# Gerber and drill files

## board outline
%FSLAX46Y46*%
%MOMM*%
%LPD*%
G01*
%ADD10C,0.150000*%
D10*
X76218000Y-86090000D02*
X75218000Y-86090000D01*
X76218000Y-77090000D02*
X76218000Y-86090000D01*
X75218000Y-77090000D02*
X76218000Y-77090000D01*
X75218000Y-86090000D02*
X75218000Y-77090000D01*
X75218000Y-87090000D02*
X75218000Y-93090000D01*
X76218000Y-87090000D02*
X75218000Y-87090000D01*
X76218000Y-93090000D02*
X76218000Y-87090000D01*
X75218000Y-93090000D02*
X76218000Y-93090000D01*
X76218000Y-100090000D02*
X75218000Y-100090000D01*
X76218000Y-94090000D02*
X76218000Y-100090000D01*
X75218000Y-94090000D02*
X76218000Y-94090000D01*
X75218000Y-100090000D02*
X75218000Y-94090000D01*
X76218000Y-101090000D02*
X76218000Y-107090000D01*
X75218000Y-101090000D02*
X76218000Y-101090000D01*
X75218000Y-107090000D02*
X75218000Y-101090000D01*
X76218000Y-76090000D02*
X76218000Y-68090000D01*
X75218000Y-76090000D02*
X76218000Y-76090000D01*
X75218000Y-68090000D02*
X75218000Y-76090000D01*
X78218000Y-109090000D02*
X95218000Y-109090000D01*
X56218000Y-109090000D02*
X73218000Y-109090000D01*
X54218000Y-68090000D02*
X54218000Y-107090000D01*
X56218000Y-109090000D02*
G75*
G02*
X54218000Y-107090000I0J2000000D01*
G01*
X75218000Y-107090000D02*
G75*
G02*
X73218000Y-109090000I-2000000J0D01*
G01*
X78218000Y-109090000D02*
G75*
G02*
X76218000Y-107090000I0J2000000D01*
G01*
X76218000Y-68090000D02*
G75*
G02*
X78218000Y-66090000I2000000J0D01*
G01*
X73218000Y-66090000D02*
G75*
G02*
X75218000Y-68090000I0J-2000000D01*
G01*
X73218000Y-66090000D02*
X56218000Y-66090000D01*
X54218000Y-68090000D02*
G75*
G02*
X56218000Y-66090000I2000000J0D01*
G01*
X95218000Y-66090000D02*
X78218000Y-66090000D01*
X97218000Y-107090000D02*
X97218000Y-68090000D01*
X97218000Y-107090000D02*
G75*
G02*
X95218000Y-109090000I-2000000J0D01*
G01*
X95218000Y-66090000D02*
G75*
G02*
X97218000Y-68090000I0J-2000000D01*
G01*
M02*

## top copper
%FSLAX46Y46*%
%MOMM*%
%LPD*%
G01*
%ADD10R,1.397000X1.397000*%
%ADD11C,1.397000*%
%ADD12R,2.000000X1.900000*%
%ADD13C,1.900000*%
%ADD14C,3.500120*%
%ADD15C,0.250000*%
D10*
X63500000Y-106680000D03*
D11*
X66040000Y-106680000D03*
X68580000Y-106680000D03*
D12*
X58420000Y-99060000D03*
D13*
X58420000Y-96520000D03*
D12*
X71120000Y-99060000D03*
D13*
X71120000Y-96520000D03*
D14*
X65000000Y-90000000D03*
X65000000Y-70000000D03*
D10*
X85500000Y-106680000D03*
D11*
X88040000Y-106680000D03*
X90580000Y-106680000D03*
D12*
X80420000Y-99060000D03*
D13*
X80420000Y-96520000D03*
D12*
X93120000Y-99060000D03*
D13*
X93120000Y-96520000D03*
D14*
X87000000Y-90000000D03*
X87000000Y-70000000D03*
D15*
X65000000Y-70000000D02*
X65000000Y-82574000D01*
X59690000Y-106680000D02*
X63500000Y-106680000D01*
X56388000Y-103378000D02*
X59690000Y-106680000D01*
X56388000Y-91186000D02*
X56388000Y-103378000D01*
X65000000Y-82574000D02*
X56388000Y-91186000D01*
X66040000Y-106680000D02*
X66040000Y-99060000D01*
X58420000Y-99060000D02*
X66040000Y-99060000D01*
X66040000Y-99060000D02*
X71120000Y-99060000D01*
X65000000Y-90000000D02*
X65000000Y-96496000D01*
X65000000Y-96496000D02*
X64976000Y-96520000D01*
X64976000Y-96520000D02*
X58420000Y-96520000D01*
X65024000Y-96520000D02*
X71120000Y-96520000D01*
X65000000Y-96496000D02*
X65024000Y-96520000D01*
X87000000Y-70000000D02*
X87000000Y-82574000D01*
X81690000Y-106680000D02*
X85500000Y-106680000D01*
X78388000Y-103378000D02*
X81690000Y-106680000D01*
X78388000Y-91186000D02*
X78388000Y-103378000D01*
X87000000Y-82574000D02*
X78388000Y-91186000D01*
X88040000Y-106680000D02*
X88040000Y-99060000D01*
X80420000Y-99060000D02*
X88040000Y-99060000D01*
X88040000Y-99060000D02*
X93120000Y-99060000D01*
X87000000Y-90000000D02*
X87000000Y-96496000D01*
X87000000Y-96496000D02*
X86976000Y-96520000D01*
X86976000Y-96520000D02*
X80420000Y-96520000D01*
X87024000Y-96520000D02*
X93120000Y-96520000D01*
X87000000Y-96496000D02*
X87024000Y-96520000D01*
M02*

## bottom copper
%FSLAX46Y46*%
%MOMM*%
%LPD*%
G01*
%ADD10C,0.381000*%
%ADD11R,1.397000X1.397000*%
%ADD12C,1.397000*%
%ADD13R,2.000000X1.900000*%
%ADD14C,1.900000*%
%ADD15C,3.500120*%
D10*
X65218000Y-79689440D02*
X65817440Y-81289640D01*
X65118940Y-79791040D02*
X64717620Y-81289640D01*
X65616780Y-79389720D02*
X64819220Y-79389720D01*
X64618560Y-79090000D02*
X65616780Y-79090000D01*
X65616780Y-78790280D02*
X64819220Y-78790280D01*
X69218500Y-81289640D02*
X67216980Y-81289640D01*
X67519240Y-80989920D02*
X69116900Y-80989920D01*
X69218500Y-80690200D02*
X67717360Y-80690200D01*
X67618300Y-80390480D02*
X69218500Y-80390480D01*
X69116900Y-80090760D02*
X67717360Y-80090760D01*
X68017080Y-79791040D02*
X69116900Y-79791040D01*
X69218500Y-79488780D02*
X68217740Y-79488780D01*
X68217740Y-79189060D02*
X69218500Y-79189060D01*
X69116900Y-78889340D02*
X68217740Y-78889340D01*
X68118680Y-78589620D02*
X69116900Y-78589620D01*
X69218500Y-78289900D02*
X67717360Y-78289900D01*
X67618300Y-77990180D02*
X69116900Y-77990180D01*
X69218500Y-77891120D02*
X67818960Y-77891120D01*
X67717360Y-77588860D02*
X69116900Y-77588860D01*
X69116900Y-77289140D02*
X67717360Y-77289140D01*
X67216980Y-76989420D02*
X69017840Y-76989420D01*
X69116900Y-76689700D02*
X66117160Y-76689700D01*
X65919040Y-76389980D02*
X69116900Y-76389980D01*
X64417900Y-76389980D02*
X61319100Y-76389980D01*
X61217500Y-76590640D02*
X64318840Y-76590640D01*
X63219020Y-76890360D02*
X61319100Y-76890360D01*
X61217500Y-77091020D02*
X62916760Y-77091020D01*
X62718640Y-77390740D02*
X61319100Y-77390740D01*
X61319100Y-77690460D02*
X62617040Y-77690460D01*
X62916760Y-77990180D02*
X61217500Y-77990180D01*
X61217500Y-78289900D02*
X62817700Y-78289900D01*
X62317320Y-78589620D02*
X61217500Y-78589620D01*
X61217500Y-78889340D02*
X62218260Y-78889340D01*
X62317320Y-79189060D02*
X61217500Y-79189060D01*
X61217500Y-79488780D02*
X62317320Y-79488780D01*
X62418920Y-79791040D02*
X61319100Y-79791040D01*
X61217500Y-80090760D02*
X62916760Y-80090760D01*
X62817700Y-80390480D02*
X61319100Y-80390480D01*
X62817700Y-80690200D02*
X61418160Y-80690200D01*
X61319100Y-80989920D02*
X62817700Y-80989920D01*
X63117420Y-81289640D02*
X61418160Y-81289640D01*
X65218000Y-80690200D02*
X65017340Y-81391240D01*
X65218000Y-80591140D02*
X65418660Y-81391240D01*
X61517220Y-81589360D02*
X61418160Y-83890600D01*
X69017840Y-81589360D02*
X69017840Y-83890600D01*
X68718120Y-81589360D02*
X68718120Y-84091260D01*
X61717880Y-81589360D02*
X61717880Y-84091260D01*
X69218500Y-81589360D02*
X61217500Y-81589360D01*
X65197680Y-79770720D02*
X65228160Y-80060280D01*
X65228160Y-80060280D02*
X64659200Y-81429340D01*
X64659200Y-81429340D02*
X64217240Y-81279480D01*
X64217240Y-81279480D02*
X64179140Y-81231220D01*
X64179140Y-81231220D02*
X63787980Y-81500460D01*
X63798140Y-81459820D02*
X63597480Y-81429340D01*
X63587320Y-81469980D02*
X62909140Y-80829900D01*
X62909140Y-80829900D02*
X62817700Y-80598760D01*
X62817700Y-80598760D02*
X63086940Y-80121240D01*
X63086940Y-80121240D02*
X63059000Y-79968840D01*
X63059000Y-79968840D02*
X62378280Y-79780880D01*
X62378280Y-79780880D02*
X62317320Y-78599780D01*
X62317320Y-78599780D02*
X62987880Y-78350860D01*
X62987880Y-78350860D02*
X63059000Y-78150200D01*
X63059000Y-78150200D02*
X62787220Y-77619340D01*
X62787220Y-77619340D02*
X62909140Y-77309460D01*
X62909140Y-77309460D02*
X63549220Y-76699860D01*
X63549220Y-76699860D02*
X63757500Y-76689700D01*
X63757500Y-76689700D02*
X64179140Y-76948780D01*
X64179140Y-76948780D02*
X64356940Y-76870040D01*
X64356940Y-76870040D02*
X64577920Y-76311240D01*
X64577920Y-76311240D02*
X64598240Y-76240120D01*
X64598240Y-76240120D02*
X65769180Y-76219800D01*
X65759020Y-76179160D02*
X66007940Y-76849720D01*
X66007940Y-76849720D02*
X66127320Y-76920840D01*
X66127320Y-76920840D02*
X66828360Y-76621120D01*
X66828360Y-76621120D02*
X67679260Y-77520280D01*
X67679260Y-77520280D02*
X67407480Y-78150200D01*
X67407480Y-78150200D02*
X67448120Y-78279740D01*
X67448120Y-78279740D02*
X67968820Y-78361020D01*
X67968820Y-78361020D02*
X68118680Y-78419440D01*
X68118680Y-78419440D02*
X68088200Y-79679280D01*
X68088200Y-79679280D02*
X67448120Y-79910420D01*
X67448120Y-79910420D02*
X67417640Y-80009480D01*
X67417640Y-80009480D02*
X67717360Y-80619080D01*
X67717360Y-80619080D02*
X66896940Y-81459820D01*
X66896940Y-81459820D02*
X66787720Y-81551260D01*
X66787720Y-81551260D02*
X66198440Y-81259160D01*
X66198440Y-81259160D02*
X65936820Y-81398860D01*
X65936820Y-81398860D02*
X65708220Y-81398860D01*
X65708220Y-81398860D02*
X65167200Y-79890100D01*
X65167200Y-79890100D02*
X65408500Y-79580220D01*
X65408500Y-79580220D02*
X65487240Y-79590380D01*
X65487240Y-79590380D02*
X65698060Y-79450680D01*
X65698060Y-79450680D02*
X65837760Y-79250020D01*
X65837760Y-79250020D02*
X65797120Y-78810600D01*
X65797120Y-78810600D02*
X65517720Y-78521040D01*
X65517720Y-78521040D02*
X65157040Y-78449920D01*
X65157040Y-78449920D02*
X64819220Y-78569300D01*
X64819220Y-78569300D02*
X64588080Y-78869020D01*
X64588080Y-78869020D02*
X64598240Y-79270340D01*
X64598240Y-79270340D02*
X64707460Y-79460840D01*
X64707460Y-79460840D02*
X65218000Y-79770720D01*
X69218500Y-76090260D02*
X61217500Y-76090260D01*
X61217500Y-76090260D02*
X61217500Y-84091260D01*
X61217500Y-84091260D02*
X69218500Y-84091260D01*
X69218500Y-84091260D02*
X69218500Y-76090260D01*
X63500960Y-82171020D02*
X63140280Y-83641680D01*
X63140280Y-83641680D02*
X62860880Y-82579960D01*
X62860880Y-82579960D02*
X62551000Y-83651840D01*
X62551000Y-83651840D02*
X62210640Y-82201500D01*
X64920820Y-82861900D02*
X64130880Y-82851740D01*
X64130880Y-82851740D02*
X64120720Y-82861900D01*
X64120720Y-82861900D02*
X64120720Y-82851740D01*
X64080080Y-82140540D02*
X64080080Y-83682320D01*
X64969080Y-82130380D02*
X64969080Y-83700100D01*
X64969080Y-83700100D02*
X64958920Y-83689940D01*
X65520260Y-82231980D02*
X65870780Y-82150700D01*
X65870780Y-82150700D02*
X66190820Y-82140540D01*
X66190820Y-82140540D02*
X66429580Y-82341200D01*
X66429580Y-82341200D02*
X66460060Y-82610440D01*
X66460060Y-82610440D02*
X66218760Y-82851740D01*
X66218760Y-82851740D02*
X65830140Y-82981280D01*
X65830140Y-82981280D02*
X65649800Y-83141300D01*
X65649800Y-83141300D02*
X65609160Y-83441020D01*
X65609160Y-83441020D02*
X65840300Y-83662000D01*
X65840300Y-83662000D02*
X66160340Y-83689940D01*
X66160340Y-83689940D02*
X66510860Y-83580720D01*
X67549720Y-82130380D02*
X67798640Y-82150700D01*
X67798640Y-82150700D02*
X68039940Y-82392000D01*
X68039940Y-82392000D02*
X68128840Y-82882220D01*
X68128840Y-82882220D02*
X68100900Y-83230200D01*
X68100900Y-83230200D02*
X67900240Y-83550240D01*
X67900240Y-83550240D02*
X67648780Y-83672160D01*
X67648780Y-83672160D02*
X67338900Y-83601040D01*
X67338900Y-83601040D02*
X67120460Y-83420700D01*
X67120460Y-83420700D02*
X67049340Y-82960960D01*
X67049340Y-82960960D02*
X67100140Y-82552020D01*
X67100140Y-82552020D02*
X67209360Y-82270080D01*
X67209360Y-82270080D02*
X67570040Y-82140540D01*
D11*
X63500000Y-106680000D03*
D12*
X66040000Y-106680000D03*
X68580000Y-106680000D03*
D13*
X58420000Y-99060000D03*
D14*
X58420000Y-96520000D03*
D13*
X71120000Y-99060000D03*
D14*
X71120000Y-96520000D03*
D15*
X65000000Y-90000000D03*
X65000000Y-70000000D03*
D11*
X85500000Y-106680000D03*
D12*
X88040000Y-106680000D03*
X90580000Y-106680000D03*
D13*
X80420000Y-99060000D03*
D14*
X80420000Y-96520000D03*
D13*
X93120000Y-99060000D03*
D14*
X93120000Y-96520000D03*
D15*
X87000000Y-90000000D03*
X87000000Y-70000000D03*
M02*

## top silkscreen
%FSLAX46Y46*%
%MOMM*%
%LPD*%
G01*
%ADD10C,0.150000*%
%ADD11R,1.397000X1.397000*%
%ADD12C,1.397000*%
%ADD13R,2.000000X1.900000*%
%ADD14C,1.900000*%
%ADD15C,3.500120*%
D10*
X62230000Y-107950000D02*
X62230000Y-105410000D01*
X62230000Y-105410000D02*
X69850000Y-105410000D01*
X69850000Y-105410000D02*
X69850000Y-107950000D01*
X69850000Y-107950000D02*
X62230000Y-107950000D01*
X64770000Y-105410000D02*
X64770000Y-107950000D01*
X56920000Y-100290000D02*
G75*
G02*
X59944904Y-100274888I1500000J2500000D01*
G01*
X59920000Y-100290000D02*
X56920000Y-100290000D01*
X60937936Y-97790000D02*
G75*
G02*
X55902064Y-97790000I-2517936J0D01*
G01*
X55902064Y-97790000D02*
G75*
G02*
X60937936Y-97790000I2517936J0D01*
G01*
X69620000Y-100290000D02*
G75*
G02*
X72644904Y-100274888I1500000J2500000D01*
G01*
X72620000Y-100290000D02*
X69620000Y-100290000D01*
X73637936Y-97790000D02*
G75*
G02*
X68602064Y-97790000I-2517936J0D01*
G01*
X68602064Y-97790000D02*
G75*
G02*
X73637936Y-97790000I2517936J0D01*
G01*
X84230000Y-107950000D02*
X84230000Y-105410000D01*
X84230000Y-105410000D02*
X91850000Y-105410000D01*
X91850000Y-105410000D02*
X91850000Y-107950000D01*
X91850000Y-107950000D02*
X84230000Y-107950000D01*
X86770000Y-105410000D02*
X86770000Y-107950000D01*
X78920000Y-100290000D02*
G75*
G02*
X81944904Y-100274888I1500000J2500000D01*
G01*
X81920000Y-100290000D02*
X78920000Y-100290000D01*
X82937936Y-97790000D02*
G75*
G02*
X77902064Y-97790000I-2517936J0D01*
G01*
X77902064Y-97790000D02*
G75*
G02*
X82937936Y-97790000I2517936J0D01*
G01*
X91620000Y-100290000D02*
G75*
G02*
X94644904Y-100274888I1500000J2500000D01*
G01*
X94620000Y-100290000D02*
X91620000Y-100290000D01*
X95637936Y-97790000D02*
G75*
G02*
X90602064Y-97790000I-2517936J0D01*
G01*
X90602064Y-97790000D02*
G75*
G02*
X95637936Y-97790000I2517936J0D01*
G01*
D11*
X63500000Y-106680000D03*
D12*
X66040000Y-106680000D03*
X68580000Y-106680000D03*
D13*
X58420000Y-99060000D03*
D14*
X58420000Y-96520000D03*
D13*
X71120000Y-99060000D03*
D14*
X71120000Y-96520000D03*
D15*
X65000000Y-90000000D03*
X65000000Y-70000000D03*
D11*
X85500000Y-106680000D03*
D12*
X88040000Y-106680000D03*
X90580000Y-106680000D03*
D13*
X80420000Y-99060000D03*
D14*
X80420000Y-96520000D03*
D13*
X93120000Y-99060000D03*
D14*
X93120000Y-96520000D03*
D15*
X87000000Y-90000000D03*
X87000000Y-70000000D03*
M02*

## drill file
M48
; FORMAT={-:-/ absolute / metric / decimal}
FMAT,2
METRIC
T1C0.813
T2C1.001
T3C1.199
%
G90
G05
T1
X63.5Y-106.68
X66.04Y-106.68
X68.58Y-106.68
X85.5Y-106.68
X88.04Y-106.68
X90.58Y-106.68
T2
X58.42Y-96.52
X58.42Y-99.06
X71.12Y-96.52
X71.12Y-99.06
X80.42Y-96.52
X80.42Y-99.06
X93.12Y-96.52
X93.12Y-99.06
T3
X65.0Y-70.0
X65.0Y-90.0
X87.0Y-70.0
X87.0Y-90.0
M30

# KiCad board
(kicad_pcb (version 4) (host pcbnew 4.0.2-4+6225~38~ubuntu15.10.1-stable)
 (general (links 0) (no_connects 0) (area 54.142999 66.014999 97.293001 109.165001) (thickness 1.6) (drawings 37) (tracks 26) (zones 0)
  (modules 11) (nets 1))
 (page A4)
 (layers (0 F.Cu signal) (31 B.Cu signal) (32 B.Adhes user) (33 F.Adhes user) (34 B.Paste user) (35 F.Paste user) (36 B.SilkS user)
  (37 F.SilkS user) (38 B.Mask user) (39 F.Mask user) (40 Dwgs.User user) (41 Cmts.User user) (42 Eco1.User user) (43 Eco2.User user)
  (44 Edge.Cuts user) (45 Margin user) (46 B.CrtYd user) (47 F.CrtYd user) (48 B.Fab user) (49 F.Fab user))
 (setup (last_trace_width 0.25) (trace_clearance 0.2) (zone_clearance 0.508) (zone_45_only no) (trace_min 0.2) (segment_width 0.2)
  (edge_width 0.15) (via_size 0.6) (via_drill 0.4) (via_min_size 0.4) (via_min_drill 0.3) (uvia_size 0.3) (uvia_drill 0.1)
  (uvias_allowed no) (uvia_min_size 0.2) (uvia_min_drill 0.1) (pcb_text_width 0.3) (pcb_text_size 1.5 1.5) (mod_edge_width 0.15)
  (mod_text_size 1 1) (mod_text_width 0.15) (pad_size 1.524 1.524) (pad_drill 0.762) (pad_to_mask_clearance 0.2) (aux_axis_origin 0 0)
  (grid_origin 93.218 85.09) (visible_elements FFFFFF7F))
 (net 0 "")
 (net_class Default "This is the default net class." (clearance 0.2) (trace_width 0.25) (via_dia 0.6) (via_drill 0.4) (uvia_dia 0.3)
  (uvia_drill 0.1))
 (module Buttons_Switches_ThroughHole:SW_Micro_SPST (layer F.Cu) (at 66.04 106.68)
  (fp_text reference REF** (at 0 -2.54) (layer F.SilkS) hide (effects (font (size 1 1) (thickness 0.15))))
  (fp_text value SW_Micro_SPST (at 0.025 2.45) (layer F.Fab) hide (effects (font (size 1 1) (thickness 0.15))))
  (fp_line (start -3.81 1.27) (end -3.81 -1.27) (layer F.SilkS) (width 0.15))
  (fp_line (start -3.81 -1.27) (end 3.81 -1.27) (layer F.SilkS) (width 0.15))
  (fp_line (start 3.81 -1.27) (end 3.81 1.27) (layer F.SilkS) (width 0.15))
  (fp_line (start 3.81 1.27) (end -3.81 1.27) (layer F.SilkS) (width 0.15))
  (fp_line (start -1.27 -1.27) (end -1.27 1.27) (layer F.SilkS) (width 0.15))
  (pad 1 thru_hole rect (at -2.54 0) (size 1.397 1.397) (drill 0.8128) (layers *.Cu *.Mask F.SilkS))
  (pad 2 thru_hole circle (at 0 0) (size 1.397 1.397) (drill 0.8128) (layers *.Cu *.Mask F.SilkS))
  (pad 3 thru_hole circle (at 2.54 0) (size 1.397 1.397) (drill 0.8128) (layers *.Cu *.Mask F.SilkS)))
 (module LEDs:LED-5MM (layer F.Cu) (at 58.42 99.06 90)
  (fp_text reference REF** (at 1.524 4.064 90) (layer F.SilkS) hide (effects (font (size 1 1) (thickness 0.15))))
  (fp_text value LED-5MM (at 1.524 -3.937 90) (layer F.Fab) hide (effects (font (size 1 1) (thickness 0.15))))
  (fp_arc (start 1.27 0) (end -1.23 -1.5) (angle 297.5) (layer F.SilkS) (width 0.15))
  (fp_line (start -1.23 1.5) (end -1.23 -1.5) (layer F.SilkS) (width 0.15))
  (fp_circle (center 1.27 0) (end 0.97 -2.5) (layer F.SilkS) (width 0.15))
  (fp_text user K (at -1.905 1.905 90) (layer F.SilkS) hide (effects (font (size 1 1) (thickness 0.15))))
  (pad 1 thru_hole rect (at 0 0 180) (size 2 1.9) (drill 1.00076) (layers *.Cu *.Mask F.SilkS))
  (pad 2 thru_hole circle (at 2.54 0 90) (size 1.9 1.9) (drill 1.00076) (layers *.Cu *.Mask F.SilkS)))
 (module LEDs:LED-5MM (layer F.Cu) (at 71.12 99.06 90)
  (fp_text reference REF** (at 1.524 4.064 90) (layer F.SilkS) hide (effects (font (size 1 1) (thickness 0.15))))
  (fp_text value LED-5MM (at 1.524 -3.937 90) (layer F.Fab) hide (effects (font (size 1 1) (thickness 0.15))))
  (fp_arc (start 1.27 0) (end -1.23 -1.5) (angle 297.5) (layer F.SilkS) (width 0.15))
  (fp_line (start -1.23 1.5) (end -1.23 -1.5) (layer F.SilkS) (width 0.15))
  (fp_circle (center 1.27 0) (end 0.97 -2.5) (layer F.SilkS) (width 0.15))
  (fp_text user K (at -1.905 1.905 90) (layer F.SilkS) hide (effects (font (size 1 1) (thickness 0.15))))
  (pad 1 thru_hole rect (at 0 0 180) (size 2 1.9) (drill 1.00076) (layers *.Cu *.Mask F.SilkS))
  (pad 2 thru_hole circle (at 2.54 0 90) (size 1.9 1.9) (drill 1.00076) (layers *.Cu *.Mask F.SilkS)))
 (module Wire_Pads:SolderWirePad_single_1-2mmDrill (layer F.Cu) (at 65 90)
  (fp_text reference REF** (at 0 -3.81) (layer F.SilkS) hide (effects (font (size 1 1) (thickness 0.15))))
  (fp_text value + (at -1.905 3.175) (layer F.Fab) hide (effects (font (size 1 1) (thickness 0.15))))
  (pad 1 thru_hole circle (at 0 0) (size 3.50012 3.50012) (drill 1.19888) (layers *.Cu *.Mask F.SilkS)))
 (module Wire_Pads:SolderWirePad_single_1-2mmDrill (layer F.Cu) (at 65 70)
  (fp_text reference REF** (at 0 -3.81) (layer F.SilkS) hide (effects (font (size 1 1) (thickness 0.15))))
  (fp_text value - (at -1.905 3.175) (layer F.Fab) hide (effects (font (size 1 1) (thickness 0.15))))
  (pad 1 thru_hole circle (at 0 0) (size 3.50012 3.50012) (drill 1.19888) (layers *.Cu *.Mask F.SilkS)))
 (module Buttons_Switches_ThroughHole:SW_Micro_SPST (layer F.Cu) (at 88.04 106.68)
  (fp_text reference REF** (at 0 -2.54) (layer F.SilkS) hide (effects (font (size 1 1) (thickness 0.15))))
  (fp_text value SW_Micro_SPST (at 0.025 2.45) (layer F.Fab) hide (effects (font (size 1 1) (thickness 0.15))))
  (fp_line (start -3.81 1.27) (end -3.81 -1.27) (layer F.SilkS) (width 0.15))
  (fp_line (start -3.81 -1.27) (end 3.81 -1.27) (layer F.SilkS) (width 0.15))
  (fp_line (start 3.81 -1.27) (end 3.81 1.27) (layer F.SilkS) (width 0.15))
  (fp_line (start 3.81 1.27) (end -3.81 1.27) (layer F.SilkS) (width 0.15))
  (fp_line (start -1.27 -1.27) (end -1.27 1.27) (layer F.SilkS) (width 0.15))
  (pad 1 thru_hole rect (at -2.54 0) (size 1.397 1.397) (drill 0.8128) (layers *.Cu *.Mask F.SilkS))
  (pad 2 thru_hole circle (at 0 0) (size 1.397 1.397) (drill 0.8128) (layers *.Cu *.Mask F.SilkS))
  (pad 3 thru_hole circle (at 2.54 0) (size 1.397 1.397) (drill 0.8128) (layers *.Cu *.Mask F.SilkS)))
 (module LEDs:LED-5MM (layer F.Cu) (at 80.42 99.06 90)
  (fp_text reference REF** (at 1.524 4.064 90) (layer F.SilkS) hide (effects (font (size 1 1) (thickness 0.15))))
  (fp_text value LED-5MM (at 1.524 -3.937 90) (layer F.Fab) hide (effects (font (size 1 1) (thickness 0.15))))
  (fp_arc (start 1.27 0) (end -1.23 -1.5) (angle 297.5) (layer F.SilkS) (width 0.15))
  (fp_line (start -1.23 1.5) (end -1.23 -1.5) (layer F.SilkS) (width 0.15))
  (fp_circle (center 1.27 0) (end 0.97 -2.5) (layer F.SilkS) (width 0.15))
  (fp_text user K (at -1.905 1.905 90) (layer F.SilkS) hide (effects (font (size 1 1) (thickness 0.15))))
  (pad 1 thru_hole rect (at 0 0 180) (size 2 1.9) (drill 1.00076) (layers *.Cu *.Mask F.SilkS))
  (pad 2 thru_hole circle (at 2.54 0 90) (size 1.9 1.9) (drill 1.00076) (layers *.Cu *.Mask F.SilkS)))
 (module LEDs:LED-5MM (layer F.Cu) (at 93.12 99.06 90)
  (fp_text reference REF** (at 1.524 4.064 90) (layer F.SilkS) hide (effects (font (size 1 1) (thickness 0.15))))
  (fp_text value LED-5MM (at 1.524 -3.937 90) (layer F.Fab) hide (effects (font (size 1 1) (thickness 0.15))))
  (fp_arc (start 1.27 0) (end -1.23 -1.5) (angle 297.5) (layer F.SilkS) (width 0.15))
  (fp_line (start -1.23 1.5) (end -1.23 -1.5) (layer F.SilkS) (width 0.15))
  (fp_circle (center 1.27 0) (end 0.97 -2.5) (layer F.SilkS) (width 0.15))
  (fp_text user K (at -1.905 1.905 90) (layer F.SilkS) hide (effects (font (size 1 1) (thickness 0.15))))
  (pad 1 thru_hole rect (at 0 0 180) (size 2 1.9) (drill 1.00076) (layers *.Cu *.Mask F.SilkS))
  (pad 2 thru_hole circle (at 2.54 0 90) (size 1.9 1.9) (drill 1.00076) (layers *.Cu *.Mask F.SilkS)))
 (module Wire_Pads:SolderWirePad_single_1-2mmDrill (layer F.Cu) (at 87 90)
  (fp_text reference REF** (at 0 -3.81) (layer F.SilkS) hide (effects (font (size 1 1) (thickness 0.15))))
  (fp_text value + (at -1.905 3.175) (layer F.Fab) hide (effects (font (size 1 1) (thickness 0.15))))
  (pad 1 thru_hole circle (at 0 0) (size 3.50012 3.50012) (drill 1.19888) (layers *.Cu *.Mask F.SilkS)))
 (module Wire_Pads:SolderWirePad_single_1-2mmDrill (layer F.Cu) (at 87 70)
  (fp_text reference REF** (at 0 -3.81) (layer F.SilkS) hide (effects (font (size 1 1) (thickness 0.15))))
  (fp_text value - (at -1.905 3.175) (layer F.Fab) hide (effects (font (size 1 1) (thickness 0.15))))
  (pad 1 thru_hole circle (at 0 0) (size 3.50012 3.50012) (drill 1.19888) (layers *.Cu *.Mask F.SilkS)))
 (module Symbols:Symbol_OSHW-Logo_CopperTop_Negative (layer B.Cu) (at 65.218 79.09 180)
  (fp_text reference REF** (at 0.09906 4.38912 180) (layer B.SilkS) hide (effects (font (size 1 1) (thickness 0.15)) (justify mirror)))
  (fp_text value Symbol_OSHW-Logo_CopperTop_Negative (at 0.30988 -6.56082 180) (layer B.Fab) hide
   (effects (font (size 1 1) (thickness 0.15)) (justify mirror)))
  (fp_line (start 0 -0.59944) (end -0.59944 -2.19964) (layer B.Cu) (width 0.381))
  (fp_line (start 0.09906 -0.70104) (end 0.50038 -2.19964) (layer B.Cu) (width 0.381))
  (fp_line (start -0.39878 -0.29972) (end 0.39878 -0.29972) (layer B.Cu) (width 0.381))
  (fp_line (start 0.59944 0) (end -0.39878 0) (layer B.Cu) (width 0.381))
  (fp_line (start -0.39878 0.29972) (end 0.39878 0.29972) (layer B.Cu) (width 0.381))
  (fp_line (start -4.0005 -2.19964) (end -1.99898 -2.19964) (layer B.Cu) (width 0.381))
  (fp_line (start -2.30124 -1.89992) (end -3.8989 -1.89992) (layer B.Cu) (width 0.381))
  (fp_line (start -4.0005 -1.6002) (end -2.49936 -1.6002) (layer B.Cu) (width 0.381))
  (fp_line (start -2.4003 -1.30048) (end -4.0005 -1.30048) (layer B.Cu) (width 0.381))
  (fp_line (start -3.8989 -1.00076) (end -2.49936 -1.00076) (layer B.Cu) (width 0.381))
  (fp_line (start -2.79908 -0.70104) (end -3.8989 -0.70104) (layer B.Cu) (width 0.381))
  (fp_line (start -4.0005 -0.39878) (end -2.99974 -0.39878) (layer B.Cu) (width 0.381))
  (fp_line (start -2.99974 -0.09906) (end -4.0005 -0.09906) (layer B.Cu) (width 0.381))
  (fp_line (start -3.8989 0.20066) (end -2.99974 0.20066) (layer B.Cu) (width 0.381))
  (fp_line (start -2.90068 0.50038) (end -3.8989 0.50038) (layer B.Cu) (width 0.381))
  (fp_line (start -4.0005 0.8001) (end -2.49936 0.8001) (layer B.Cu) (width 0.381))
  (fp_line (start -2.4003 1.09982) (end -3.8989 1.09982) (layer B.Cu) (width 0.381))
  (fp_line (start -4.0005 1.19888) (end -2.60096 1.19888) (layer B.Cu) (width 0.381))
  (fp_line (start -2.49936 1.50114) (end -3.8989 1.50114) (layer B.Cu) (width 0.381))
  (fp_line (start -3.8989 1.80086) (end -2.49936 1.80086) (layer B.Cu) (width 0.381))
  (fp_line (start -1.99898 2.10058) (end -3.79984 2.10058) (layer B.Cu) (width 0.381))
  (fp_line (start -3.8989 2.4003) (end -0.89916 2.4003) (layer B.Cu) (width 0.381))
  (fp_line (start -0.70104 2.70002) (end -3.8989 2.70002) (layer B.Cu) (width 0.381))
  (fp_line (start 0.8001 2.70002) (end 3.8989 2.70002) (layer B.Cu) (width 0.381))
  (fp_line (start 4.0005 2.49936) (end 0.89916 2.49936) (layer B.Cu) (width 0.381))
  (fp_line (start 1.99898 2.19964) (end 3.8989 2.19964) (layer B.Cu) (width 0.381))
  (fp_line (start 4.0005 1.99898) (end 2.30124 1.99898) (layer B.Cu) (width 0.381))
  (fp_line (start 2.49936 1.69926) (end 3.8989 1.69926) (layer B.Cu) (width 0.381))
  (fp_line (start 3.8989 1.39954) (end 2.60096 1.39954) (layer B.Cu) (width 0.381))
  (fp_line (start 2.30124 1.09982) (end 4.0005 1.09982) (layer B.Cu) (width 0.381))
  (fp_line (start 4.0005 0.8001) (end 2.4003 0.8001) (layer B.Cu) (width 0.381))
  (fp_line (start 2.90068 0.50038) (end 4.0005 0.50038) (layer B.Cu) (width 0.381))
  (fp_line (start 4.0005 0.20066) (end 2.99974 0.20066) (layer B.Cu) (width 0.381))
  (fp_line (start 2.90068 -0.09906) (end 4.0005 -0.09906) (layer B.Cu) (width 0.381))
  (fp_line (start 4.0005 -0.39878) (end 2.90068 -0.39878) (layer B.Cu) (width 0.381))
  (fp_line (start 2.79908 -0.70104) (end 3.8989 -0.70104) (layer B.Cu) (width 0.381))
  (fp_line (start 4.0005 -1.00076) (end 2.30124 -1.00076) (layer B.Cu) (width 0.381))
  (fp_line (start 2.4003 -1.30048) (end 3.8989 -1.30048) (layer B.Cu) (width 0.381))
  (fp_line (start 2.4003 -1.6002) (end 3.79984 -1.6002) (layer B.Cu) (width 0.381))
  (fp_line (start 3.8989 -1.89992) (end 2.4003 -1.89992) (layer B.Cu) (width 0.381))
  (fp_line (start 2.10058 -2.19964) (end 3.79984 -2.19964) (layer B.Cu) (width 0.381))
  (fp_line (start 0 -1.6002) (end 0.20066 -2.30124) (layer B.Cu) (width 0.381))
  (fp_line (start 0 -1.50114) (end -0.20066 -2.30124) (layer B.Cu) (width 0.381))
  (fp_line (start 3.70078 -2.49936) (end 3.79984 -4.8006) (layer B.Cu) (width 0.381))
  (fp_line (start -3.79984 -2.49936) (end -3.79984 -4.8006) (layer B.Cu) (width 0.381))
  (fp_line (start -3.50012 -2.49936) (end -3.50012 -5.00126) (layer B.Cu) (width 0.381))
  (fp_line (start 3.50012 -2.49936) (end 3.50012 -5.00126) (layer B.Cu) (width 0.381))
  (fp_line (start -4.0005 -2.49936) (end 4.0005 -2.49936) (layer B.Cu) (width 0.381))
  (fp_line (start 0.02032 -0.68072) (end -0.01016 -0.97028) (layer B.Cu) (width 0.381))
  (fp_line (start -0.01016 -0.97028) (end 0.5588 -2.33934) (layer B.Cu) (width 0.381))
  (fp_line (start 0.5588 -2.33934) (end 1.00076 -2.18948) (layer B.Cu) (width 0.381))
  (fp_line (start 1.00076 -2.18948) (end 1.03886 -2.14122) (layer B.Cu) (width 0.381))
  (fp_line (start 1.03886 -2.14122) (end 1.43002 -2.41046) (layer B.Cu) (width 0.381))
  (fp_line (start 1.41986 -2.36982) (end 1.62052 -2.33934) (layer B.Cu) (width 0.381))
  (fp_line (start 1.63068 -2.37998) (end 2.30886 -1.7399) (layer B.Cu) (width 0.381))
  (fp_line (start 2.30886 -1.7399) (end 2.4003 -1.50876) (layer B.Cu) (width 0.381))
  (fp_line (start 2.4003 -1.50876) (end 2.13106 -1.03124) (layer B.Cu) (width 0.381))
  (fp_line (start 2.13106 -1.03124) (end 2.159 -0.87884) (layer B.Cu) (width 0.381))
  (fp_line (start 2.159 -0.87884) (end 2.83972 -0.69088) (layer B.Cu) (width 0.381))
  (fp_line (start 2.83972 -0.69088) (end 2.90068 0.49022) (layer B.Cu) (width 0.381))
  (fp_line (start 2.90068 0.49022) (end 2.23012 0.73914) (layer B.Cu) (width 0.381))
  (fp_line (start 2.23012 0.73914) (end 2.159 0.9398) (layer B.Cu) (width 0.381))
  (fp_line (start 2.159 0.9398) (end 2.43078 1.47066) (layer B.Cu) (width 0.381))
  (fp_line (start 2.43078 1.47066) (end 2.30886 1.78054) (layer B.Cu) (width 0.381))
  (fp_line (start 2.30886 1.78054) (end 1.66878 2.39014) (layer B.Cu) (width 0.381))
  (fp_line (start 1.66878 2.39014) (end 1.4605 2.4003) (layer B.Cu) (width 0.381))
  (fp_line (start 1.4605 2.4003) (end 1.03886 2.14122) (layer B.Cu) (width 0.381))
  (fp_line (start 1.03886 2.14122) (end 0.86106 2.21996) (layer B.Cu) (width 0.381))
  (fp_line (start 0.86106 2.21996) (end 0.64008 2.77876) (layer B.Cu) (width 0.381))
  (fp_line (start 0.64008 2.77876) (end 0.61976 2.84988) (layer B.Cu) (width 0.381))
  (fp_line (start 0.61976 2.84988) (end -0.55118 2.8702) (layer B.Cu) (width 0.381))
  (fp_line (start -0.54102 2.91084) (end -0.78994 2.24028) (layer B.Cu) (width 0.381))
  (fp_line (start -0.78994 2.24028) (end -0.90932 2.16916) (layer B.Cu) (width 0.381))
  (fp_line (start -0.90932 2.16916) (end -1.61036 2.46888) (layer B.Cu) (width 0.381))
  (fp_line (start -1.61036 2.46888) (end -2.46126 1.56972) (layer B.Cu) (width 0.381))
  (fp_line (start -2.46126 1.56972) (end -2.18948 0.9398) (layer B.Cu) (width 0.381))
  (fp_line (start -2.18948 0.9398) (end -2.23012 0.81026) (layer B.Cu) (width 0.381))
  (fp_line (start -2.23012 0.81026) (end -2.75082 0.72898) (layer B.Cu) (width 0.381))
  (fp_line (start -2.75082 0.72898) (end -2.90068 0.67056) (layer B.Cu) (width 0.381))
  (fp_line (start -2.90068 0.67056) (end -2.8702 -0.58928) (layer B.Cu) (width 0.381))
  (fp_line (start -2.8702 -0.58928) (end -2.23012 -0.82042) (layer B.Cu) (width 0.381))
  (fp_line (start -2.23012 -0.82042) (end -2.19964 -0.91948) (layer B.Cu) (width 0.381))
  (fp_line (start -2.19964 -0.91948) (end -2.49936 -1.52908) (layer B.Cu) (width 0.381))
  (fp_line (start -2.49936 -1.52908) (end -1.67894 -2.36982) (layer B.Cu) (width 0.381))
  (fp_line (start -1.67894 -2.36982) (end -1.56972 -2.46126) (layer B.Cu) (width 0.381))
  (fp_line (start -1.56972 -2.46126) (end -0.98044 -2.16916) (layer B.Cu) (width 0.381))
  (fp_line (start -0.98044 -2.16916) (end -0.71882 -2.30886) (layer B.Cu) (width 0.381))
  (fp_line (start -0.71882 -2.30886) (end -0.49022 -2.30886) (layer B.Cu) (width 0.381))
  (fp_line (start -0.49022 -2.30886) (end 0.0508 -0.8001) (layer B.Cu) (width 0.381))
  (fp_line (start 0.0508 -0.8001) (end -0.1905 -0.49022) (layer B.Cu) (width 0.381))
  (fp_line (start -0.1905 -0.49022) (end -0.26924 -0.50038) (layer B.Cu) (width 0.381))
  (fp_line (start -0.26924 -0.50038) (end -0.48006 -0.36068) (layer B.Cu) (width 0.381))
  (fp_line (start -0.48006 -0.36068) (end -0.61976 -0.16002) (layer B.Cu) (width 0.381))
  (fp_line (start -0.61976 -0.16002) (end -0.57912 0.2794) (layer B.Cu) (width 0.381))
  (fp_line (start -0.57912 0.2794) (end -0.29972 0.56896) (layer B.Cu) (width 0.381))
  (fp_line (start -0.29972 0.56896) (end 0.06096 0.64008) (layer B.Cu) (width 0.381))
  (fp_line (start 0.06096 0.64008) (end 0.39878 0.5207) (layer B.Cu) (width 0.381))
  (fp_line (start 0.39878 0.5207) (end 0.62992 0.22098) (layer B.Cu) (width 0.381))
  (fp_line (start 0.62992 0.22098) (end 0.61976 -0.18034) (layer B.Cu) (width 0.381))
  (fp_line (start 0.61976 -0.18034) (end 0.51054 -0.37084) (layer B.Cu) (width 0.381))
  (fp_line (start 0.51054 -0.37084) (end 0 -0.68072) (layer B.Cu) (width 0.381))
  (fp_line (start -4.0005 2.99974) (end 4.0005 2.99974) (layer B.Cu) (width 0.381))
  (fp_line (start 4.0005 2.99974) (end 4.0005 -5.00126) (layer B.Cu) (width 0.381))
  (fp_line (start 4.0005 -5.00126) (end -4.0005 -5.00126) (layer B.Cu) (width 0.381))
  (fp_line (start -4.0005 -5.00126) (end -4.0005 2.99974) (layer B.Cu) (width 0.381))
  (fp_line (start 1.71704 -3.08102) (end 2.07772 -4.55168) (layer B.Cu) (width 0.381))
  (fp_line (start 2.07772 -4.55168) (end 2.35712 -3.48996) (layer B.Cu) (width 0.381))
  (fp_line (start 2.35712 -3.48996) (end 2.667 -4.56184) (layer B.Cu) (width 0.381))
  (fp_line (start 2.667 -4.56184) (end 3.00736 -3.1115) (layer B.Cu) (width 0.381))
  (fp_line (start 0.29718 -3.7719) (end 1.08712 -3.76174) (layer B.Cu) (width 0.381))
  (fp_line (start 1.08712 -3.76174) (end 1.09728 -3.7719) (layer B.Cu) (width 0.381))
  (fp_line (start 1.09728 -3.7719) (end 1.09728 -3.76174) (layer B.Cu) (width 0.381))
  (fp_line (start 1.13792 -3.05054) (end 1.13792 -4.59232) (layer B.Cu) (width 0.381))
  (fp_line (start 0.24892 -3.04038) (end 0.24892 -4.6101) (layer B.Cu) (width 0.381))
  (fp_line (start 0.24892 -4.6101) (end 0.25908 -4.59994) (layer B.Cu) (width 0.381))
  (fp_line (start -0.30226 -3.14198) (end -0.65278 -3.0607) (layer B.Cu) (width 0.381))
  (fp_line (start -0.65278 -3.0607) (end -0.97282 -3.05054) (layer B.Cu) (width 0.381))
  (fp_line (start -0.97282 -3.05054) (end -1.21158 -3.2512) (layer B.Cu) (width 0.381))
  (fp_line (start -1.21158 -3.2512) (end -1.24206 -3.52044) (layer B.Cu) (width 0.381))
  (fp_line (start -1.24206 -3.52044) (end -1.00076 -3.76174) (layer B.Cu) (width 0.381))
  (fp_line (start -1.00076 -3.76174) (end -0.61214 -3.89128) (layer B.Cu) (width 0.381))
  (fp_line (start -0.61214 -3.89128) (end -0.4318 -4.0513) (layer B.Cu) (width 0.381))
  (fp_line (start -0.4318 -4.0513) (end -0.39116 -4.35102) (layer B.Cu) (width 0.381))
  (fp_line (start -0.39116 -4.35102) (end -0.6223 -4.572) (layer B.Cu) (width 0.381))
  (fp_line (start -0.6223 -4.572) (end -0.94234 -4.59994) (layer B.Cu) (width 0.381))
  (fp_line (start -0.94234 -4.59994) (end -1.29286 -4.49072) (layer B.Cu) (width 0.381))
  (fp_line (start -2.33172 -3.04038) (end -2.58064 -3.0607) (layer B.Cu) (width 0.381))
  (fp_line (start -2.58064 -3.0607) (end -2.82194 -3.302) (layer B.Cu) (width 0.381))
  (fp_line (start -2.82194 -3.302) (end -2.91084 -3.79222) (layer B.Cu) (width 0.381))
  (fp_line (start -2.91084 -3.79222) (end -2.8829 -4.1402) (layer B.Cu) (width 0.381))
  (fp_line (start -2.8829 -4.1402) (end -2.68224 -4.46024) (layer B.Cu) (width 0.381))
  (fp_line (start -2.68224 -4.46024) (end -2.43078 -4.58216) (layer B.Cu) (width 0.381))
  (fp_line (start -2.43078 -4.58216) (end -2.1209 -4.51104) (layer B.Cu) (width 0.381))
  (fp_line (start -2.1209 -4.51104) (end -1.90246 -4.3307) (layer B.Cu) (width 0.381))
  (fp_line (start -1.90246 -4.3307) (end -1.83134 -3.87096) (layer B.Cu) (width 0.381))
  (fp_line (start -1.83134 -3.87096) (end -1.88214 -3.46202) (layer B.Cu) (width 0.381))
  (fp_line (start -1.88214 -3.46202) (end -1.99136 -3.18008) (layer B.Cu) (width 0.381))
  (fp_line (start -1.99136 -3.18008) (end -2.35204 -3.05054) (layer B.Cu) (width 0.381)))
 (gr_line (start 76.218 86.09) (end 75.218 86.09) (angle 90) (layer Edge.Cuts) (width 0.15))
 (gr_line (start 76.218 77.09) (end 76.218 86.09) (angle 90) (layer Edge.Cuts) (width 0.15))
 (gr_line (start 75.218 77.09) (end 76.218 77.09) (angle 90) (layer Edge.Cuts) (width 0.15))
 (gr_line (start 75.218 86.09) (end 75.218 77.09) (angle 90) (layer Edge.Cuts) (width 0.15))
 (gr_line (start 75.218 87.09) (end 75.218 93.09) (angle 90) (layer Edge.Cuts) (width 0.15))
 (gr_line (start 76.218 87.09) (end 75.218 87.09) (angle 90) (layer Edge.Cuts) (width 0.15))
 (gr_line (start 76.218 93.09) (end 76.218 87.09) (angle 90) (layer Edge.Cuts) (width 0.15))
 (gr_line (start 75.218 93.09) (end 76.218 93.09) (angle 90) (layer Edge.Cuts) (width 0.15))
 (gr_line (start 76.218 100.09) (end 75.218 100.09) (angle 90) (layer Edge.Cuts) (width 0.15))
 (gr_line (start 76.218 94.09) (end 76.218 100.09) (angle 90) (layer Edge.Cuts) (width 0.15))
 (gr_line (start 75.218 94.09) (end 76.218 94.09) (angle 90) (layer Edge.Cuts) (width 0.15))
 (gr_line (start 75.218 100.09) (end 75.218 94.09) (angle 90) (layer Edge.Cuts) (width 0.15))
 (gr_line (start 76.218 101.09) (end 76.218 107.09) (angle 90) (layer Edge.Cuts) (width 0.15))
 (gr_line (start 75.218 101.09) (end 76.218 101.09) (angle 90) (layer Edge.Cuts) (width 0.15))
 (gr_line (start 75.218 107.09) (end 75.218 101.09) (angle 90) (layer Edge.Cuts) (width 0.15))
 (gr_line (start 76.218 76.09) (end 76.218 68.09) (angle 90) (layer Edge.Cuts) (width 0.15))
 (gr_line (start 75.218 76.09) (end 76.218 76.09) (angle 90) (layer Edge.Cuts) (width 0.15))
 (gr_line (start 75.218 68.09) (end 75.218 76.09) (angle 90) (layer Edge.Cuts) (width 0.15))
 (gr_line (start 78.218 109.09) (end 95.218 109.09) (angle 90) (layer Edge.Cuts) (width 0.15))
 (gr_line (start 56.218 109.09) (end 73.218 109.09) (angle 90) (layer Edge.Cuts) (width 0.15))
 (gr_line (start 54.218 68.09) (end 54.218 107.09) (angle 90) (layer Edge.Cuts) (width 0.15))
 (gr_arc (start 56.218 107.09) (end 56.218 109.09) (angle 90) (layer Edge.Cuts) (width 0.15))
 (gr_arc (start 73.218 107.09) (end 75.218 107.09) (angle 90) (layer Edge.Cuts) (width 0.15))
 (gr_arc (start 78.218 107.09) (end 78.218 109.09) (angle 90) (layer Edge.Cuts) (width 0.15))
 (gr_arc (start 78.218 68.09) (end 76.218 68.09) (angle 90) (layer Edge.Cuts) (width 0.15))
 (gr_arc (start 73.218 68.09) (end 73.218 66.09) (angle 90) (layer Edge.Cuts) (width 0.15))
 (gr_line (start 73.218 66.09) (end 56.218 66.09) (angle 90) (layer Edge.Cuts) (width 0.15))
 (gr_arc (start 56.218 68.09) (end 54.218 68.09) (angle 90) (layer Edge.Cuts) (width 0.15))
 (gr_line (start 95.218 66.09) (end 78.218 66.09) (angle 90) (layer Edge.Cuts) (width 0.15))
 (gr_line (start 97.218 107.09) (end 97.218 68.09) (angle 90) (layer Edge.Cuts) (width 0.15))
 (gr_arc (start 95.218 107.09) (end 97.218 107.09) (angle 90) (layer Edge.Cuts) (width 0.15))
 (gr_arc (start 95.218 68.09) (end 95.218 66.09) (angle 90) (layer Edge.Cuts) (width 0.15))
 (segment (start 65 70) (end 65 82.574) (width 0.25) (layer F.Cu) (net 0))
 (segment (start 59.69 106.68) (end 63.5 106.68) (width 0.25) (layer F.Cu) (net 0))
 (segment (start 56.388 103.378) (end 59.69 106.68) (width 0.25) (layer F.Cu) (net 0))
 (segment (start 56.388 91.186) (end 56.388 103.378) (width 0.25) (layer F.Cu) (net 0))
 (segment (start 65 82.574) (end 56.388 91.186) (width 0.25) (layer F.Cu) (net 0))
 (segment (start 66.04 106.68) (end 66.04 99.06) (width 0.25) (layer F.Cu) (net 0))
 (segment (start 58.42 99.06) (end 66.04 99.06) (width 0.25) (layer F.Cu) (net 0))
 (segment (start 66.04 99.06) (end 71.12 99.06) (width 0.25) (layer F.Cu) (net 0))
 (segment (start 65 90) (end 65 96.496) (width 0.25) (layer F.Cu) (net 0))
 (segment (start 65 96.496) (end 64.976 96.52) (width 0.25) (layer F.Cu) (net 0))
 (segment (start 64.976 96.52) (end 58.42 96.52) (width 0.25) (layer F.Cu) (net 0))
 (segment (start 65.024 96.52) (end 71.12 96.52) (width 0.25) (layer F.Cu) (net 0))
 (segment (start 65 96.496) (end 65.024 96.52) (width 0.25) (layer F.Cu) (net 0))
 (segment (start 87 70) (end 87 82.574) (width 0.25) (layer F.Cu) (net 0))
 (segment (start 81.69 106.68) (end 85.5 106.68) (width 0.25) (layer F.Cu) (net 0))
 (segment (start 78.388 103.378) (end 81.69 106.68) (width 0.25) (layer F.Cu) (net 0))
 (segment (start 78.388 91.186) (end 78.388 103.378) (width 0.25) (layer F.Cu) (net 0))
 (segment (start 87 82.574) (end 78.388 91.186) (width 0.25) (layer F.Cu) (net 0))
 (segment (start 88.04 106.68) (end 88.04 99.06) (width 0.25) (layer F.Cu) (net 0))
 (segment (start 80.42 99.06) (end 88.04 99.06) (width 0.25) (layer F.Cu) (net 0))
 (segment (start 88.04 99.06) (end 93.12 99.06) (width 0.25) (layer F.Cu) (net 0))
 (segment (start 87 90) (end 87 96.496) (width 0.25) (layer F.Cu) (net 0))
 (segment (start 87 96.496) (end 86.976 96.52) (width 0.25) (layer F.Cu) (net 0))
 (segment (start 86.976 96.52) (end 80.42 96.52) (width 0.25) (layer F.Cu) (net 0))
 (segment (start 87.024 96.52) (end 93.12 96.52) (width 0.25) (layer F.Cu) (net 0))
 (segment (start 87 96.496) (end 87.024 96.52) (width 0.25) (layer F.Cu) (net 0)))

